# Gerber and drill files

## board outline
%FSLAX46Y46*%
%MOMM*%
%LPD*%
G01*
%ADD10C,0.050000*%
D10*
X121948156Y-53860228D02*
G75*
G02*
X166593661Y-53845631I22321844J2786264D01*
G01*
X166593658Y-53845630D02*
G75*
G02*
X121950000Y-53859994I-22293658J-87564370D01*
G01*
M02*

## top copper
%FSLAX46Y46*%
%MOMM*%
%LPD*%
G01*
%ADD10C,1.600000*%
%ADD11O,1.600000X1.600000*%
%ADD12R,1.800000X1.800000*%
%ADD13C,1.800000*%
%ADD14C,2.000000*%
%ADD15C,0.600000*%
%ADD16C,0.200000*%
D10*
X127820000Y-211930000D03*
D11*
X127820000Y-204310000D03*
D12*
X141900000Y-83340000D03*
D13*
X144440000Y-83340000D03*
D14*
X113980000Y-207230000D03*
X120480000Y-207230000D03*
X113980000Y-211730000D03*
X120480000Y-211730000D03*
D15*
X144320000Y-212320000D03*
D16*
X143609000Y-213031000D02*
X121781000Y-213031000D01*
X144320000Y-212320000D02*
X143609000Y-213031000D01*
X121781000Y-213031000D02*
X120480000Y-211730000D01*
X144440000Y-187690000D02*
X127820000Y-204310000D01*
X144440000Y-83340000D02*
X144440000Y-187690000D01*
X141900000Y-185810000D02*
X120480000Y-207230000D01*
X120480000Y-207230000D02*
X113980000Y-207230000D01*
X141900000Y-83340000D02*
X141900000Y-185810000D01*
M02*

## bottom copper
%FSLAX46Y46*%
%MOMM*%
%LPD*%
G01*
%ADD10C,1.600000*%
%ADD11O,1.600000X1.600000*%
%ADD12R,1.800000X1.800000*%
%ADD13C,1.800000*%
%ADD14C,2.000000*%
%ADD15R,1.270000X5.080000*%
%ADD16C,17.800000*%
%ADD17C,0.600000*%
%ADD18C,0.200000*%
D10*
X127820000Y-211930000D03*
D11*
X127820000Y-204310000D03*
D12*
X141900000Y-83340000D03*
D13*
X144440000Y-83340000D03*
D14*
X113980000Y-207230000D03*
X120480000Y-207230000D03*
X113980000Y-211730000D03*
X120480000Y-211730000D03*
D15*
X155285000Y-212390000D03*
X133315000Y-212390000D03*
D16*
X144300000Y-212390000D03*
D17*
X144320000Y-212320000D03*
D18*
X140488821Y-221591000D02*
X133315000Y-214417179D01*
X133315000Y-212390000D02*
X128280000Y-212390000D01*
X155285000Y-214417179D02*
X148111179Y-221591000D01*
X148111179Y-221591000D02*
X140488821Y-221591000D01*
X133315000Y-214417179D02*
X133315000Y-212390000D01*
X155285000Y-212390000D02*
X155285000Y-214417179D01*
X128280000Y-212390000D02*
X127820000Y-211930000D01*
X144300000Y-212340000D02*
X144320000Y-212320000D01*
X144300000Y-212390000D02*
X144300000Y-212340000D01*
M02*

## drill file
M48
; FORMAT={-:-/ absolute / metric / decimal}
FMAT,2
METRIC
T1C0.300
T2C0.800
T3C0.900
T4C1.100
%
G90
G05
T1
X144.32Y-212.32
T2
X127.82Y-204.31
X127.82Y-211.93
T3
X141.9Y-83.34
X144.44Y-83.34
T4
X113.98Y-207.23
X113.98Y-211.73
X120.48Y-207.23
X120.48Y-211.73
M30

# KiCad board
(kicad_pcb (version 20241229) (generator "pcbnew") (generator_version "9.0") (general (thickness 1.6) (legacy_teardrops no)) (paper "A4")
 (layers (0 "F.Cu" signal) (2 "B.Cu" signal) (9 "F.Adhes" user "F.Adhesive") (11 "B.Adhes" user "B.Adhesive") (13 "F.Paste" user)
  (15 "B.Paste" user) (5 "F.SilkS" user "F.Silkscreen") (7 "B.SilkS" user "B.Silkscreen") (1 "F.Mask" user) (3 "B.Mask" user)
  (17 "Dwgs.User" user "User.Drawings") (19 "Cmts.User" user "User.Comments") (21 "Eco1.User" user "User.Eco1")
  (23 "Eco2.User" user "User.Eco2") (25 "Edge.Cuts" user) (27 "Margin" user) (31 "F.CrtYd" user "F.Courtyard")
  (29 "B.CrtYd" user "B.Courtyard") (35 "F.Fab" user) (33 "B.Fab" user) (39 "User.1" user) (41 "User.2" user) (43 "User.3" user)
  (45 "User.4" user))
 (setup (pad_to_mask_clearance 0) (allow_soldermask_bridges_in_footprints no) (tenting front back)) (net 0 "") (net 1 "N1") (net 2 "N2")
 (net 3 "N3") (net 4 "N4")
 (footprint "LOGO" (layer "F.Cu") (at 144.3 141.41)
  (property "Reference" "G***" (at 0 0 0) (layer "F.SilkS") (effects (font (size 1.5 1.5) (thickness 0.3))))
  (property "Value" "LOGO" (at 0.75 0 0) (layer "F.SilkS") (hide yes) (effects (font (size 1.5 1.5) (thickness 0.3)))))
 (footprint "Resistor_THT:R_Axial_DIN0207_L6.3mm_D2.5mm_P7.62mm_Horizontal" (layer "F.Cu") (at 127.82 211.93 90)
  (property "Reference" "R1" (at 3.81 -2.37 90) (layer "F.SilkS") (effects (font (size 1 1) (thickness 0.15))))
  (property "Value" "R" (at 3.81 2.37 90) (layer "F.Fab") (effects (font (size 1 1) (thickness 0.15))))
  (pad "1" thru_hole circle (at 0 0 90) (size 1.6 1.6) (drill 0.8) (layers "*.Cu" "*.Mask") (remove_unused_layers no) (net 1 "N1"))
  (pad "2" thru_hole oval (at 7.62 0 90) (size 1.6 1.6) (drill 0.8) (layers "*.Cu" "*.Mask") (remove_unused_layers no) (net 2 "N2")))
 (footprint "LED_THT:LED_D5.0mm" (layer "F.Cu") (at 141.9 83.34)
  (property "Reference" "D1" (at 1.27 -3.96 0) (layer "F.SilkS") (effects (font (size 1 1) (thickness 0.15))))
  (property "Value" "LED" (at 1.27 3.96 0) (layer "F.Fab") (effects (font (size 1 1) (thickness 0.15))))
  (pad "1" thru_hole rect (at 0 0) (size 1.8 1.8) (drill 0.9) (layers "*.Cu" "*.Mask") (remove_unused_layers no) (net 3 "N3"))
  (pad "2" thru_hole circle (at 2.54 0) (size 1.8 1.8) (drill 0.9) (layers "*.Cu" "*.Mask") (remove_unused_layers no) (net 2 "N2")))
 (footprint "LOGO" (layer "F.Cu") (at 146.39 95.76)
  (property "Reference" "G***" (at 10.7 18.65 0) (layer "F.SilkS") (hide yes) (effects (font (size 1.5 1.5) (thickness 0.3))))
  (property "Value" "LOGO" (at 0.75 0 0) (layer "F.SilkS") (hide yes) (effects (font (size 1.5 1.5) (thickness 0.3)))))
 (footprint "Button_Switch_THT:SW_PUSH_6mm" (layer "F.Cu") (at 113.98 207.23)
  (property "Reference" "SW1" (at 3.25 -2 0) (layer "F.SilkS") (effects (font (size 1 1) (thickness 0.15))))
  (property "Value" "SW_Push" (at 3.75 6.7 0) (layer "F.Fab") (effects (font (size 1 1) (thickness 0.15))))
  (pad "1" thru_hole circle (at 0 0 90) (size 2 2) (drill 1.1) (layers "*.Cu" "*.Mask") (remove_unused_layers no) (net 3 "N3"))
  (pad "1" thru_hole circle (at 6.5 0 90) (size 2 2) (drill 1.1) (layers "*.Cu" "*.Mask") (remove_unused_layers no) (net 3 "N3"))
  (pad "2" thru_hole circle (at 0 4.5 90) (size 2 2) (drill 1.1) (layers "*.Cu" "*.Mask") (remove_unused_layers no) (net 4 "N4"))
  (pad "2" thru_hole circle (at 6.5 4.5 90) (size 2 2) (drill 1.1) (layers "*.Cu" "*.Mask") (remove_unused_layers no) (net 4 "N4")))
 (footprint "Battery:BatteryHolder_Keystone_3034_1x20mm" (layer "B.Cu") (at 144.3 212.39 180)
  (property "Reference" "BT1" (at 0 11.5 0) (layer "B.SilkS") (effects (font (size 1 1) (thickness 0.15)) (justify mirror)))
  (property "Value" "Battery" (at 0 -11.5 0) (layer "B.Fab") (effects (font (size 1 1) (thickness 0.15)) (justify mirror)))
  (pad "1" smd rect (at -10.985 0 180) (size 1.27 5.08) (layers "B.Cu" "B.Mask" "B.Paste") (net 1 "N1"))
  (pad "1" smd rect (at 10.985 0 180) (size 1.27 5.08) (layers "B.Cu" "B.Mask" "B.Paste") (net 1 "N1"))
  (pad "2" smd circle (at 0 0 180) (size 17.8 17.8) (layers "B.Cu" "B.Mask") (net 4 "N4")))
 (gr_arc (start 121.948156 53.860228) (mid 144.262645 28.5789) (end 166.593661 53.845631) (stroke (width 0.05) (type default))
  (layer "Edge.Cuts"))
 (gr_arc (start 166.593658 53.84563) (mid 144.329072 231.767762) (end 121.95 53.859994) (stroke (width 0.05) (type default))
  (layer "Edge.Cuts"))
 (segment (start 140.488821 221.591) (end 133.315 214.417179) (width 0.2) (layer "B.Cu") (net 1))
 (segment (start 133.315 212.39) (end 128.28 212.39) (width 0.2) (layer "B.Cu") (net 1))
 (segment (start 155.285 214.417179) (end 148.111179 221.591) (width 0.2) (layer "B.Cu") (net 1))
 (segment (start 148.111179 221.591) (end 140.488821 221.591) (width 0.2) (layer "B.Cu") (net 1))
 (segment (start 133.315 214.417179) (end 133.315 212.39) (width 0.2) (layer "B.Cu") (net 1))
 (segment (start 155.285 212.39) (end 155.285 214.417179) (width 0.2) (layer "B.Cu") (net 1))
 (segment (start 128.28 212.39) (end 127.82 211.93) (width 0.2) (layer "B.Cu") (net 1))
 (segment (start 143.609 213.031) (end 121.781 213.031) (width 0.2) (layer "F.Cu") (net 4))
 (segment (start 144.32 212.32) (end 143.609 213.031) (width 0.2) (layer "F.Cu") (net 4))
 (segment (start 121.781 213.031) (end 120.48 211.73) (width 0.2) (layer "F.Cu") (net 4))
 (via (at 144.32 212.32) (size 0.6) (drill 0.3) (layers "F.Cu" "B.Cu") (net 4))
 (segment (start 144.3 212.34) (end 144.32 212.32) (width 0.2) (layer "B.Cu") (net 4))
 (segment (start 144.3 212.39) (end 144.3 212.34) (width 0.2) (layer "B.Cu") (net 4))
 (segment (start 144.44 187.69) (end 127.82 204.31) (width 0.2) (layer "F.Cu") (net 2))
 (segment (start 144.44 83.34) (end 144.44 187.69) (width 0.2) (layer "F.Cu") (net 2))
 (segment (start 141.9 185.81) (end 120.48 207.23) (width 0.2) (layer "F.Cu") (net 3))
 (segment (start 120.48 207.23) (end 113.98 207.23) (width 0.2) (layer "F.Cu") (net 3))
 (segment (start 141.9 83.34) (end 141.9 185.81) (width 0.2) (layer "F.Cu") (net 3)))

